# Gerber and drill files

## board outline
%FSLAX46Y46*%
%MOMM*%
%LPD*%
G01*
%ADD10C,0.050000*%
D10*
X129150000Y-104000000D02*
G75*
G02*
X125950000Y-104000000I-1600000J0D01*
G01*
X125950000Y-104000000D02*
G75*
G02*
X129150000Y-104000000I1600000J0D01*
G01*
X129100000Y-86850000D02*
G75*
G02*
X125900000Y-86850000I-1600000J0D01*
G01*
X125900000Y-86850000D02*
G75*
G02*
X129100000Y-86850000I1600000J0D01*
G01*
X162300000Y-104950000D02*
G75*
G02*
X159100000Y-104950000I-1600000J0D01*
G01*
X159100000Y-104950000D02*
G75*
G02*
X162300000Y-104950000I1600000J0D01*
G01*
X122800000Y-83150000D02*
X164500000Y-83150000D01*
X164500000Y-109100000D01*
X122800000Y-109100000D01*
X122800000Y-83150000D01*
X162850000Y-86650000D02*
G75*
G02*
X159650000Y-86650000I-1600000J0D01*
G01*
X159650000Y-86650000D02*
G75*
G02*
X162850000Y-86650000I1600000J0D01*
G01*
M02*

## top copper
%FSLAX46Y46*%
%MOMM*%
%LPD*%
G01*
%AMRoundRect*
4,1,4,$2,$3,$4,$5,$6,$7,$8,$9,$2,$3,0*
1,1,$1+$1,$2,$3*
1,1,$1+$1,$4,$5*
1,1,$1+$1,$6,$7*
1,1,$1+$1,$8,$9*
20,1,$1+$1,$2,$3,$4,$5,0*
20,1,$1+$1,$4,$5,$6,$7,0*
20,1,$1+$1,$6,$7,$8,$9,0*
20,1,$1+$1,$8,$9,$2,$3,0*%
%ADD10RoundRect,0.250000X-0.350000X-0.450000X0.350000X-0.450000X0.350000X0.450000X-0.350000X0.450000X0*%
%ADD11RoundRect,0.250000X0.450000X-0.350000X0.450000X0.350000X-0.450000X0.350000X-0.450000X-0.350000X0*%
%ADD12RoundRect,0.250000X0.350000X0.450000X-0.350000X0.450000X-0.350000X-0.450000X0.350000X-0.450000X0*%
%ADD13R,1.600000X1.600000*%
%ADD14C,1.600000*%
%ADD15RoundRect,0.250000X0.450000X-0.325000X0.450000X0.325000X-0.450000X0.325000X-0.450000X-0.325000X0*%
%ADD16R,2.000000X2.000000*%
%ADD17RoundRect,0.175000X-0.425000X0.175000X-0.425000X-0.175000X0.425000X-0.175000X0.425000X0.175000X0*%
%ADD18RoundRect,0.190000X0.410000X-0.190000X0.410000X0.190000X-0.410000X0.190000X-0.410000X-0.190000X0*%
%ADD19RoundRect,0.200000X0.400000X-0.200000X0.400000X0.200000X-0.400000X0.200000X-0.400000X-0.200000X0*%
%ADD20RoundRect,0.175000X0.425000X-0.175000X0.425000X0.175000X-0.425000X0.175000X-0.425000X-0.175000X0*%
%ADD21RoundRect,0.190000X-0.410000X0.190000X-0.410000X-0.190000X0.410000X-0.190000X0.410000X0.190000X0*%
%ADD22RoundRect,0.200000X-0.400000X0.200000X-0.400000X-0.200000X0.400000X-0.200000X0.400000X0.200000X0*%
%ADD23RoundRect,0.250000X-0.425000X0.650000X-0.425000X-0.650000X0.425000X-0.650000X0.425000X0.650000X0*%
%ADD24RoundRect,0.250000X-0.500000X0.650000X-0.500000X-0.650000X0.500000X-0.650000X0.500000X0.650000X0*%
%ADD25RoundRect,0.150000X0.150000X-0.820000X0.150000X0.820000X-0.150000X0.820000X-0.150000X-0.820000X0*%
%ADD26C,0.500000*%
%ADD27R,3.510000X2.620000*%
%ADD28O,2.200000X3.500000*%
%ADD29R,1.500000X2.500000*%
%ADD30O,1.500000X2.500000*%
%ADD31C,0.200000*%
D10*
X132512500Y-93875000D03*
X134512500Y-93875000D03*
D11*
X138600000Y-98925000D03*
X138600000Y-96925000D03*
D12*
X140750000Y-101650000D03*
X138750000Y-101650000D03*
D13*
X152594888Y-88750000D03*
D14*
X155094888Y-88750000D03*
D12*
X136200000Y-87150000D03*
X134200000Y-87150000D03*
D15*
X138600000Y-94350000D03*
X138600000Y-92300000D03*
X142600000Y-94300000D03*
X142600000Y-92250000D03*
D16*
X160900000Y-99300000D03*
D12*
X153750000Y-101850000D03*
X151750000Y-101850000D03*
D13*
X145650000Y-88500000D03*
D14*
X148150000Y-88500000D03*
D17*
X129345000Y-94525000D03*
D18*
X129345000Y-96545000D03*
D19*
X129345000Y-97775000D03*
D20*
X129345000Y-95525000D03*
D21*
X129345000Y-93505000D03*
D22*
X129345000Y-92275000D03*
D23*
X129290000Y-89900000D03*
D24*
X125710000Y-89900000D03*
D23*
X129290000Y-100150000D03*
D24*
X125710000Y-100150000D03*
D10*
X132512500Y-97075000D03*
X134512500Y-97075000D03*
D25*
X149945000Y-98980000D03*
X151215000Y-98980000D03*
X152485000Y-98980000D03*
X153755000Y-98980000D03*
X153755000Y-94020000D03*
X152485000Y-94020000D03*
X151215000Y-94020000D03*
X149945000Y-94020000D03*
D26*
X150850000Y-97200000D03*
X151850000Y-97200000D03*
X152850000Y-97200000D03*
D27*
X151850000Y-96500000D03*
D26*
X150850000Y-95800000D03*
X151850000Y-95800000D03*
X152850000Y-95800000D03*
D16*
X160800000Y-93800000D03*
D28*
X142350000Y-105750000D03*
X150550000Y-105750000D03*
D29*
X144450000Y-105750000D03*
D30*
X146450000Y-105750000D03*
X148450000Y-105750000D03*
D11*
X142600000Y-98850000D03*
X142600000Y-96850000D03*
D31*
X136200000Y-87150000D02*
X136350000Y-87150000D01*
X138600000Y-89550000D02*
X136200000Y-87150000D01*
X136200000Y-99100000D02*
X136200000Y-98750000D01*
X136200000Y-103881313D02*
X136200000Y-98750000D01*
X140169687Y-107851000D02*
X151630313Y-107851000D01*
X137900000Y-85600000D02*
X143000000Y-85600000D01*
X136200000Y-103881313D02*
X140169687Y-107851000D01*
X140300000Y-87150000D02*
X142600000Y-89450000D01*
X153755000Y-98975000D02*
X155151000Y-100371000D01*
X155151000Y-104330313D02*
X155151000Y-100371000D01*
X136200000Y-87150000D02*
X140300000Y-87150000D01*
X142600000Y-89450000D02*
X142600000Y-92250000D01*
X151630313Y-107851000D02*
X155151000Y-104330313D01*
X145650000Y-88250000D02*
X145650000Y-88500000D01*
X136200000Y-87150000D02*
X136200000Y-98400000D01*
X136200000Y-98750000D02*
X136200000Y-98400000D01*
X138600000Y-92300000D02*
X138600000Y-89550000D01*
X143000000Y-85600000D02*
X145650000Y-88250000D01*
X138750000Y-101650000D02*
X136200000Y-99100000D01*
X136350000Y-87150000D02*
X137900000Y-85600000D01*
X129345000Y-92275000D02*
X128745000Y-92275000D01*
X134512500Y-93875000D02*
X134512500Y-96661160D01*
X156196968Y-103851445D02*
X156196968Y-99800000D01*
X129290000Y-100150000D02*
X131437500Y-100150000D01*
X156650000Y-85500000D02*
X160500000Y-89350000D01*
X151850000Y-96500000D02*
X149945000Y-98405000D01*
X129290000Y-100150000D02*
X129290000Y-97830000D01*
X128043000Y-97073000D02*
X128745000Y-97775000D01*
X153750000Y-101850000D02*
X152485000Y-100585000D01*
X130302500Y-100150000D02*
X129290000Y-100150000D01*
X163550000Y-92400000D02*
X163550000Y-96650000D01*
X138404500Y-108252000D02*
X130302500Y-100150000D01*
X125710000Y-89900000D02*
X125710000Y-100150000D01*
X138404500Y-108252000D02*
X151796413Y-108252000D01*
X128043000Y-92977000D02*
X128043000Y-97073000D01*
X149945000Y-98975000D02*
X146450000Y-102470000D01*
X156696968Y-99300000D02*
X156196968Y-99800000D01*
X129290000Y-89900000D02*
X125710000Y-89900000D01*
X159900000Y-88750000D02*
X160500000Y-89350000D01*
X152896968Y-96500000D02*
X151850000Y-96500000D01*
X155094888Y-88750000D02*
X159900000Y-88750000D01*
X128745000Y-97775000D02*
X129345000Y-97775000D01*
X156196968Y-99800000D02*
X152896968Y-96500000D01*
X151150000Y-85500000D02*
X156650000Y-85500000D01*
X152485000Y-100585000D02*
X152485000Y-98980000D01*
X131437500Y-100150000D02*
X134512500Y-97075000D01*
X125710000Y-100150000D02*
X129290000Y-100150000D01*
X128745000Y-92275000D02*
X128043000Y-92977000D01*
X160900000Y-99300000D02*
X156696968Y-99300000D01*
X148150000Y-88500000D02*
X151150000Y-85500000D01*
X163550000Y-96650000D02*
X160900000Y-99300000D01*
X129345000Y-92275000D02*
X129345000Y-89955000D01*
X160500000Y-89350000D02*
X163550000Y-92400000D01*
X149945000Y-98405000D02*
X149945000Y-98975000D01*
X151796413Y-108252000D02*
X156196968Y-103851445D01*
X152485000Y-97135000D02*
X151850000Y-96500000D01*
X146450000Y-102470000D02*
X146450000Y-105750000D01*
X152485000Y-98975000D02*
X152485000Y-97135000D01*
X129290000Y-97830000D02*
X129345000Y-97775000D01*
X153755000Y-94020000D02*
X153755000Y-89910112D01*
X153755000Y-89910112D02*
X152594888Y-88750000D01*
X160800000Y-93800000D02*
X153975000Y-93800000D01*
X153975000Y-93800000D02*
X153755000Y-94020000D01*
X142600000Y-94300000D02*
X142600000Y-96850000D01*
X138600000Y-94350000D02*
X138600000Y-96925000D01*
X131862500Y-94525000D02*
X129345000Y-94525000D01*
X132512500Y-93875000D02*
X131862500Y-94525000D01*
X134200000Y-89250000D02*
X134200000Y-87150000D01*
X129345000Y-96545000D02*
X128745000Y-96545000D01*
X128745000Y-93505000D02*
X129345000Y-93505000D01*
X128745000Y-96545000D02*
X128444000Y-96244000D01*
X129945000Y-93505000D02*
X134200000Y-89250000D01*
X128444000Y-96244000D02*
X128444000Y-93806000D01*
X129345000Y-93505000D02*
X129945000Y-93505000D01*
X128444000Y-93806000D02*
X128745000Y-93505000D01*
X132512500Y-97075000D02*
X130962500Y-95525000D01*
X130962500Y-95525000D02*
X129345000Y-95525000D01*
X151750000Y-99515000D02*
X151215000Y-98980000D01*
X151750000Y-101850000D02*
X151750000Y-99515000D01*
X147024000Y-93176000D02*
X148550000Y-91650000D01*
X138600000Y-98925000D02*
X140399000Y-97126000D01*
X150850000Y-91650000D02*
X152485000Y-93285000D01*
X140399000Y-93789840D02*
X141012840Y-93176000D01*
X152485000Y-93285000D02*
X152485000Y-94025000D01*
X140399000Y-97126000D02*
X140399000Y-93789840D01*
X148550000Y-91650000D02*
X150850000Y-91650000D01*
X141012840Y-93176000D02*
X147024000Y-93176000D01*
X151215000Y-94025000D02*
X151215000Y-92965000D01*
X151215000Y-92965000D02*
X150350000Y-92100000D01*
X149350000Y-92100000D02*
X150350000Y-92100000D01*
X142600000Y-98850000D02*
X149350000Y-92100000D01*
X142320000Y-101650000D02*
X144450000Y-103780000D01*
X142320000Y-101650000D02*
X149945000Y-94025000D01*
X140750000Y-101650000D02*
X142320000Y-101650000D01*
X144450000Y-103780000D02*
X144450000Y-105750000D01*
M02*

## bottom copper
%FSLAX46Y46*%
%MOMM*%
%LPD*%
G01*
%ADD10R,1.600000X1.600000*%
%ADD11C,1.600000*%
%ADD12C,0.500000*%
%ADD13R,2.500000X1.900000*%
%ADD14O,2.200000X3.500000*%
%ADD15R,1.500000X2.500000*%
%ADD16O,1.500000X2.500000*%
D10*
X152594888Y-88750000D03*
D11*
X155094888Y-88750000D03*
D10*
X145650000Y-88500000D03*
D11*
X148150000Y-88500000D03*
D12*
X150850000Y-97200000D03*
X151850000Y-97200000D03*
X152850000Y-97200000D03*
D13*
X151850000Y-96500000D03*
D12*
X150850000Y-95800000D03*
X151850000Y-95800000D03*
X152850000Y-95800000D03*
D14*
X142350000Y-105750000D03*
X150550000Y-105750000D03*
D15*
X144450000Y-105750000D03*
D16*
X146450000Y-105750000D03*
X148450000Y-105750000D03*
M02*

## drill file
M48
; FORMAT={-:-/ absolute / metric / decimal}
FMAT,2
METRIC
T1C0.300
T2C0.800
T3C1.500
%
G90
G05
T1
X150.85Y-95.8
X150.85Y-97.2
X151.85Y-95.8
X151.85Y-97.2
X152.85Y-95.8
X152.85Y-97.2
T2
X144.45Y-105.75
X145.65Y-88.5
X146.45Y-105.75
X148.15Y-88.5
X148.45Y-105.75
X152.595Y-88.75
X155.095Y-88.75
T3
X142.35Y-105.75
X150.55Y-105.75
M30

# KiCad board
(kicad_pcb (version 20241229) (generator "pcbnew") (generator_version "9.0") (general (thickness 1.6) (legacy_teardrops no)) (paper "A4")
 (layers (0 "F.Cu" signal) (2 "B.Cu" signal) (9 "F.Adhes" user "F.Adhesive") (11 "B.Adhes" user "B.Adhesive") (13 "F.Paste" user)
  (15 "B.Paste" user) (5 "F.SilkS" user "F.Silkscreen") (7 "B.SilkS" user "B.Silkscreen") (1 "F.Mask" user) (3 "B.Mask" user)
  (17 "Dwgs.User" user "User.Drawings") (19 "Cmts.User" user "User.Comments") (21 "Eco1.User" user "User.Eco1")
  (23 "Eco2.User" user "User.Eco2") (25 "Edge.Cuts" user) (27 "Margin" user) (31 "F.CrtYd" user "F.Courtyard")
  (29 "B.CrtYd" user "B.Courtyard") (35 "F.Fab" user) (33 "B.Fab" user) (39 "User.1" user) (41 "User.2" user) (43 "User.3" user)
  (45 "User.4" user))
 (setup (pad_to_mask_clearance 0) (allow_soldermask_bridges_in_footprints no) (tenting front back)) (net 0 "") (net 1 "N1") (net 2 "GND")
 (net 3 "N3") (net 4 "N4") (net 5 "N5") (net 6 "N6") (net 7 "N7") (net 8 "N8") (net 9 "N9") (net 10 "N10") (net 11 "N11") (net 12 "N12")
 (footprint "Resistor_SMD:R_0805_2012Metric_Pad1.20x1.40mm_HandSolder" (layer "F.Cu") (at 133.5125 93.875)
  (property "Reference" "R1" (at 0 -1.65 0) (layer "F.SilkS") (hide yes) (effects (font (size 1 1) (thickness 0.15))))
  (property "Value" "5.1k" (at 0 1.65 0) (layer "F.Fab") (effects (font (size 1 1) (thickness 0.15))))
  (pad "1" smd roundrect (at -1 0) (size 1.2 1.4) (layers "F.Cu" "F.Mask" "F.Paste") (roundrect_rratio 0.208333) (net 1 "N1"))
  (pad "2" smd roundrect (at 1 0) (size 1.2 1.4) (layers "F.Cu" "F.Mask" "F.Paste") (roundrect_rratio 0.208333) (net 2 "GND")))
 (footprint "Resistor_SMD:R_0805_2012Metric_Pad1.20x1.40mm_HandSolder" (layer "F.Cu") (at 138.6 97.925 90)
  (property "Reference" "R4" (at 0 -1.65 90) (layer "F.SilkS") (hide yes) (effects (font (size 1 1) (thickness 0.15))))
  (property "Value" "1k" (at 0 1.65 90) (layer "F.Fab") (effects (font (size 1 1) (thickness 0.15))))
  (pad "1" smd roundrect (at -1 0 90) (size 1.2 1.4) (layers "F.Cu" "F.Mask" "F.Paste") (roundrect_rratio 0.208333) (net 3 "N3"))
  (pad "2" smd roundrect (at 1 0 90) (size 1.2 1.4) (layers "F.Cu" "F.Mask" "F.Paste") (roundrect_rratio 0.208333) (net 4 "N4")))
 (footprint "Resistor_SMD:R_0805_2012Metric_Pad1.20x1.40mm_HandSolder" (layer "F.Cu") (at 139.75 101.65 180)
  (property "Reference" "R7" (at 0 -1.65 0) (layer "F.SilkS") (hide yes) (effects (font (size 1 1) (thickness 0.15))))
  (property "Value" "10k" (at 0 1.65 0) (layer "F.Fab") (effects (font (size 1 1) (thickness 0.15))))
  (pad "1" smd roundrect (at -1 0 180) (size 1.2 1.4) (layers "F.Cu" "F.Mask" "F.Paste") (roundrect_rratio 0.208333) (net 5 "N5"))
  (pad "2" smd roundrect (at 1 0 180) (size 1.2 1.4) (layers "F.Cu" "F.Mask" "F.Paste") (roundrect_rratio 0.208333) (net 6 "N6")))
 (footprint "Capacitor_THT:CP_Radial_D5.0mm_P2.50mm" (layer "F.Cu") (at 152.594888 88.75)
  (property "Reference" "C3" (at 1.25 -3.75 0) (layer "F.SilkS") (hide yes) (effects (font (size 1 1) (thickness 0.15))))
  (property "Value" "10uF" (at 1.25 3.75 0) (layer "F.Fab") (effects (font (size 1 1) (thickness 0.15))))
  (pad "1" thru_hole rect (at 0 0) (size 1.6 1.6) (drill 0.8) (layers "*.Cu" "*.Mask") (remove_unused_layers no) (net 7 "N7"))
  (pad "2" thru_hole circle (at 2.5 0) (size 1.6 1.6) (drill 0.8) (layers "*.Cu" "*.Mask") (remove_unused_layers no) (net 2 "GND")))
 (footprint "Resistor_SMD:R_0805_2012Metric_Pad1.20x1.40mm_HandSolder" (layer "F.Cu") (at 135.2 87.15 180)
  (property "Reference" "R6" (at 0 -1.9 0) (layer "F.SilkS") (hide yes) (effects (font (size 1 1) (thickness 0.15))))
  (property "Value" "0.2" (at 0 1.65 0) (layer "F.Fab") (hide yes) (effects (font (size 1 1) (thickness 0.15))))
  (pad "1" smd roundrect (at -1 0 180) (size 1.2 1.4) (layers "F.Cu" "F.Mask" "F.Paste") (roundrect_rratio 0.208333) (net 6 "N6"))
  (pad "2" smd roundrect (at 1 0 180) (size 1.2 1.4) (layers "F.Cu" "F.Mask" "F.Paste") (roundrect_rratio 0.208333) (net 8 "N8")))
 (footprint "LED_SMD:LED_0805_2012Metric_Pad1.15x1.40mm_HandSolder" (layer "F.Cu") (at 138.6 93.325 90)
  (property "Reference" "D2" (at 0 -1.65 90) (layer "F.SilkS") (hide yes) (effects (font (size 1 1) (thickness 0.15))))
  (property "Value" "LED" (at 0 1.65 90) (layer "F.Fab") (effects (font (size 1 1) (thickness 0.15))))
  (pad "1" smd roundrect (at -1.025 0 90) (size 1.15 1.4) (layers "F.Cu" "F.Mask" "F.Paste") (roundrect_rratio 0.217391) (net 4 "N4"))
  (pad "2" smd roundrect (at 1.025 0 90) (size 1.15 1.4) (layers "F.Cu" "F.Mask" "F.Paste") (roundrect_rratio 0.217391) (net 6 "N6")))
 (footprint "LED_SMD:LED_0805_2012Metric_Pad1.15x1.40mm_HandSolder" (layer "F.Cu") (at 142.6 93.275 90)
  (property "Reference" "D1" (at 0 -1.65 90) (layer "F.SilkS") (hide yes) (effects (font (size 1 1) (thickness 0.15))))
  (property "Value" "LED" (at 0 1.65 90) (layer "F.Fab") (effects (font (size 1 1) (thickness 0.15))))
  (pad "1" smd roundrect (at -1.025 0 90) (size 1.15 1.4) (layers "F.Cu" "F.Mask" "F.Paste") (roundrect_rratio 0.217391) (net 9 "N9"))
  (pad "2" smd roundrect (at 1.025 0 90) (size 1.15 1.4) (layers "F.Cu" "F.Mask" "F.Paste") (roundrect_rratio 0.217391) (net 6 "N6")))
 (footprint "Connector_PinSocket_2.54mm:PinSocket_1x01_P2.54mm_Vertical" (layer "F.Cu") (at 160.9 99.3)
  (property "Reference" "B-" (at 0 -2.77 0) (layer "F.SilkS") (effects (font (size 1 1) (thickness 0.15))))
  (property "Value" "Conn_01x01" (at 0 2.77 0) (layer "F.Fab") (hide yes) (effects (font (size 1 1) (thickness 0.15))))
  (pad "1" smd rect (at 0 0) (size 2 2) (layers "F.Cu" "F.Mask" "F.Paste") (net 2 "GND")))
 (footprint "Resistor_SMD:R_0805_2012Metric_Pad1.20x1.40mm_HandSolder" (layer "F.Cu") (at 152.75 101.85 180)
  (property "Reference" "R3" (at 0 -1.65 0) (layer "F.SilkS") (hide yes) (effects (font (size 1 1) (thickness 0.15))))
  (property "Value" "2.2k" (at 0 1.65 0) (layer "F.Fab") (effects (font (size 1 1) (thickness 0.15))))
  (pad "1" smd roundrect (at -1 0 180) (size 1.2 1.4) (layers "F.Cu" "F.Mask" "F.Paste") (roundrect_rratio 0.208333) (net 2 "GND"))
  (pad "2" smd roundrect (at 1 0 180) (size 1.2 1.4) (layers "F.Cu" "F.Mask" "F.Paste") (roundrect_rratio 0.208333) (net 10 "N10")))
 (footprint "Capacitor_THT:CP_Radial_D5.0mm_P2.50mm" (layer "F.Cu") (at 145.65 88.5)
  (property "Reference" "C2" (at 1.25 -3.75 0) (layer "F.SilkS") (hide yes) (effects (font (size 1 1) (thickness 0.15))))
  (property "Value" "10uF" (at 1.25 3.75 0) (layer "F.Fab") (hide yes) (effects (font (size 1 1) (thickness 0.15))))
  (pad "1" thru_hole rect (at 0 0) (size 1.6 1.6) (drill 0.8) (layers "*.Cu" "*.Mask") (remove_unused_layers no) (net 6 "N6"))
  (pad "2" thru_hole circle (at 2.5 0) (size 1.6 1.6) (drill 0.8) (layers "*.Cu" "*.Mask") (remove_unused_layers no) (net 2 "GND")))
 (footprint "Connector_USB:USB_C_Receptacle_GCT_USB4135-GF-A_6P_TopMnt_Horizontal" (layer "F.Cu") (at 126.3125 95.025 -90)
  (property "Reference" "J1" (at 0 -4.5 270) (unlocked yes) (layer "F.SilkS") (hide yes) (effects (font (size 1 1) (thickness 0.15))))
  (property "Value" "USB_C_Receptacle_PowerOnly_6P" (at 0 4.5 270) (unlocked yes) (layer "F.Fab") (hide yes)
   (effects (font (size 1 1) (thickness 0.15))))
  (pad "A5" smd roundrect (at -0.5 -3.0325 270) (size 0.7 1.2) (layers "F.Cu" "F.Mask" "F.Paste") (roundrect_rratio 0.25) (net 1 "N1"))
  (pad "A9" smd roundrect (at 1.52 -3.0325 90) (size 0.76 1.2) (layers "F.Cu" "F.Mask" "F.Paste") (roundrect_rratio 0.25) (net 8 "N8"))
  (pad "A12" smd roundrect (at 2.75 -3.0325 90) (size 0.8 1.2) (layers "F.Cu" "F.Mask" "F.Paste") (roundrect_rratio 0.25) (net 2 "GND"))
  (pad "B5" smd roundrect (at 0.5 -3.0325 90) (size 0.7 1.2) (layers "F.Cu" "F.Mask" "F.Paste") (roundrect_rratio 0.25) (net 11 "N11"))
  (pad "B9" smd roundrect (at -1.52 -3.0325 270) (size 0.76 1.2) (layers "F.Cu" "F.Mask" "F.Paste") (roundrect_rratio 0.25) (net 8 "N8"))
  (pad "B12" smd roundrect (at -2.75 -3.0325 270) (size 0.8 1.2) (layers "F.Cu" "F.Mask" "F.Paste") (roundrect_rratio 0.25) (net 2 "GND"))
  (pad "S1" smd roundrect (at -5.125 -2.9775 270) (size 1.8 1.35) (layers "F.Cu" "F.Mask" "F.Paste") (roundrect_rratio 0.1851851852)
   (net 2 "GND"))
  (pad "S1" smd roundrect (at -5.125 0.6025 270) (size 1.8 1.5) (layers "F.Cu" "F.Mask" "F.Paste") (roundrect_rratio 0.1666666667)
   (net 2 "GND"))
  (pad "S1" smd roundrect (at 5.125 -2.9775 270) (size 1.8 1.35) (layers "F.Cu" "F.Mask" "F.Paste") (roundrect_rratio 0.1851851852)
   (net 2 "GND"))
  (pad "S1" smd roundrect (at 5.125 0.6025 270) (size 1.8 1.5) (layers "F.Cu" "F.Mask" "F.Paste") (roundrect_rratio 0.1666666667)
   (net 2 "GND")))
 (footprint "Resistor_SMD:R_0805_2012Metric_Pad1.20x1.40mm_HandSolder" (layer "F.Cu") (at 133.5125 97.075)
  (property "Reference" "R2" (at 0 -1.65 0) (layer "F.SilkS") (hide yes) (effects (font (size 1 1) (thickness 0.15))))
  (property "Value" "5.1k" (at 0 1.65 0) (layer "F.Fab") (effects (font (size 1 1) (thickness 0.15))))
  (pad "1" smd roundrect (at -1 0) (size 1.2 1.4) (layers "F.Cu" "F.Mask" "F.Paste") (roundrect_rratio 0.208333) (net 11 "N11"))
  (pad "2" smd roundrect (at 1 0) (size 1.2 1.4) (layers "F.Cu" "F.Mask" "F.Paste") (roundrect_rratio 0.208333) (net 2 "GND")))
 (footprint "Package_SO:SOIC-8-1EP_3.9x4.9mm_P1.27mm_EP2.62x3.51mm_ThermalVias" (layer "F.Cu") (at 151.85 96.5 90)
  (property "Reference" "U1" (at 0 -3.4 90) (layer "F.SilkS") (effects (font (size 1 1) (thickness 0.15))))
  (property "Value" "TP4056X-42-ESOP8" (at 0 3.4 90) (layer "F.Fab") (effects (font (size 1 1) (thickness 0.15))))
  (pad "" smd roundrect (at -0.655 -0.875 90) (size 1.1 1.47) (layers "F.Paste") (roundrect_rratio 0.227273))
  (pad "" smd roundrect (at -0.655 0.875 90) (size 1.1 1.47) (layers "F.Paste") (roundrect_rratio 0.227273))
  (pad "" smd roundrect (at 0.655 -0.875 90) (size 1.1 1.47) (layers "F.Paste") (roundrect_rratio 0.227273))
  (pad "" smd roundrect (at 0.655 0.875 90) (size 1.1 1.47) (layers "F.Paste") (roundrect_rratio 0.227273))
  (pad "1" smd roundrect (at -2.48 -1.905 90) (size 1.94 0.6) (layers "F.Cu" "F.Mask" "F.Paste") (roundrect_rratio 0.25) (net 2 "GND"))
  (pad "2" smd roundrect (at -2.48 -0.635 90) (size 1.94 0.6) (layers "F.Cu" "F.Mask" "F.Paste") (roundrect_rratio 0.25) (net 10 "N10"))
  (pad "3" smd roundrect (at -2.48 0.635 90) (size 1.94 0.6) (layers "F.Cu" "F.Mask" "F.Paste") (roundrect_rratio 0.25) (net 2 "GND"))
  (pad "4" smd roundrect (at -2.48 1.905 90) (size 1.94 0.6) (layers "F.Cu" "F.Mask" "F.Paste") (roundrect_rratio 0.25) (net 6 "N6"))
  (pad "5" smd roundrect (at 2.48 1.905 90) (size 1.94 0.6) (layers "F.Cu" "F.Mask" "F.Paste") (roundrect_rratio 0.25) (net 7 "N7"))
  (pad "6" smd roundrect (at 2.48 0.635 90) (size 1.94 0.6) (layers "F.Cu" "F.Mask" "F.Paste") (roundrect_rratio 0.25) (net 3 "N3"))
  (pad "7" smd roundrect (at 2.48 -0.635 90) (size 1.94 0.6) (layers "F.Cu" "F.Mask" "F.Paste") (roundrect_rratio 0.25) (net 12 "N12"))
  (pad "8" smd roundrect (at 2.48 -1.905 90) (size 1.94 0.6) (layers "F.Cu" "F.Mask" "F.Paste") (roundrect_rratio 0.25) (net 5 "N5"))
  (pad "9" thru_hole circle (at -0.7 -1 90) (size 0.5 0.5) (drill 0.3) (layers "*.Cu") (remove_unused_layers no) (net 2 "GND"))
  (pad "9" thru_hole circle (at -0.7 0 90) (size 0.5 0.5) (drill 0.3) (layers "*.Cu") (remove_unused_layers no) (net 2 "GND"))
  (pad "9" thru_hole circle (at -0.7 1 90) (size 0.5 0.5) (drill 0.3) (layers "*.Cu") (remove_unused_layers no) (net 2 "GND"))
  (pad "9" smd rect (at 0 0 90) (size 1.9 2.5) (layers "B.Cu") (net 2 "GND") (zone_connect 2))
  (pad "9" smd rect (at 0 0 90) (size 2.62 3.51) (layers "F.Cu" "F.Mask") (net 2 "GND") (zone_connect 2))
  (pad "9" thru_hole circle (at 0.7 -1 90) (size 0.5 0.5) (drill 0.3) (layers "*.Cu") (remove_unused_layers no) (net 2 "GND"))
  (pad "9" thru_hole circle (at 0.7 0 90) (size 0.5 0.5) (drill 0.3) (layers "*.Cu") (remove_unused_layers no) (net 2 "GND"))
  (pad "9" thru_hole circle (at 0.7 1 90) (size 0.5 0.5) (drill 0.3) (layers "*.Cu") (remove_unused_layers no) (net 2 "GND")))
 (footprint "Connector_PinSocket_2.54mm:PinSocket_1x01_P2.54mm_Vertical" (layer "F.Cu") (at 160.8 93.8)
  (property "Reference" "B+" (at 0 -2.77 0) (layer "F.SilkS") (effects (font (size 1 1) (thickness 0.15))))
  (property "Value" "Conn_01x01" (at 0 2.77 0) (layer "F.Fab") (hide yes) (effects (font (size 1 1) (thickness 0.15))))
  (pad "1" smd rect (at 0 0) (size 2 2) (layers "F.Cu" "F.Mask" "F.Paste") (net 7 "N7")))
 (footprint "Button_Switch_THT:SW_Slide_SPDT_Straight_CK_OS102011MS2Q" (layer "F.Cu") (at 144.45 105.75)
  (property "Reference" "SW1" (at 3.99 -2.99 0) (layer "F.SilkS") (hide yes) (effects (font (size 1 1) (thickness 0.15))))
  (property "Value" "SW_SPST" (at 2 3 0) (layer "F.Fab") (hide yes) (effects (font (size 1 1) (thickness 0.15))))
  (pad "" thru_hole oval (at -2.1 0) (size 2.2 3.5) (drill 1.5) (layers "*.Cu" "*.Mask") (remove_unused_layers no))
  (pad "" thru_hole oval (at 6.1 0) (size 2.2 3.5) (drill 1.5) (layers "*.Cu" "*.Mask") (remove_unused_layers no))
  (pad "1" thru_hole rect (at 0 0) (size 1.5 2.5) (drill 0.8) (layers "*.Cu" "*.Mask") (remove_unused_layers no) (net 5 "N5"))
  (pad "2" thru_hole oval (at 2 0) (size 1.5 2.5) (drill 0.8) (layers "*.Cu" "*.Mask") (remove_unused_layers no) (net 2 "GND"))
  (pad "3" thru_hole oval (at 4 0) (size 1.5 2.5) (drill 0.8) (layers "*.Cu" "*.Mask") (remove_unused_layers no)))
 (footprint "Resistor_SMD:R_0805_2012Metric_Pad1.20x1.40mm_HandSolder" (layer "F.Cu") (at 142.6 97.85 90)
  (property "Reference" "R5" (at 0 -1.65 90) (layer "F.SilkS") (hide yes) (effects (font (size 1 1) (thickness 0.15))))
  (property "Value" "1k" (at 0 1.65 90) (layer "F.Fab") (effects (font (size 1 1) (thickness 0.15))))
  (pad "1" smd roundrect (at -1 0 90) (size 1.2 1.4) (layers "F.Cu" "F.Mask" "F.Paste") (roundrect_rratio 0.208333) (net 12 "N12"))
  (pad "2" smd roundrect (at 1 0 90) (size 1.2 1.4) (layers "F.Cu" "F.Mask" "F.Paste") (roundrect_rratio 0.208333) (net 9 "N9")))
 (gr_circle (center 127.55 104) (end 127.55 105.6) (stroke (width 0.05) (type default)) (fill no) (layer "Edge.Cuts"))
 (gr_circle (center 127.5 86.85) (end 127.5 88.45) (stroke (width 0.05) (type default)) (fill no) (layer "Edge.Cuts"))
 (gr_circle (center 160.7 104.95) (end 160.7 106.55) (stroke (width 0.05) (type default)) (fill no) (layer "Edge.Cuts"))
 (gr_rect (start 122.8 83.15) (end 164.5 109.1) (stroke (width 0.05) (type default)) (fill no) (layer "Edge.Cuts"))
 (gr_circle (center 161.25 86.65) (end 161.25 88.25) (stroke (width 0.05) (type default)) (fill no) (layer "Edge.Cuts"))
 (segment (start 136.2 87.15) (end 136.35 87.15) (width 0.2) (layer "F.Cu") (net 6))
 (segment (start 138.6 89.55) (end 136.2 87.15) (width 0.2) (layer "F.Cu") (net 6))
 (segment (start 136.2 99.1) (end 136.2 98.75) (width 0.2) (layer "F.Cu") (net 6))
 (segment (start 136.2 103.881313) (end 136.2 98.75) (width 0.2) (layer "F.Cu") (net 6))
 (segment (start 140.169687 107.851) (end 151.630313 107.851) (width 0.2) (layer "F.Cu") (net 6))
 (segment (start 137.9 85.6) (end 143 85.6) (width 0.2) (layer "F.Cu") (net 6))
 (segment (start 136.2 103.881313) (end 140.169687 107.851) (width 0.2) (layer "F.Cu") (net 6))
 (segment (start 140.3 87.15) (end 142.6 89.45) (width 0.2) (layer "F.Cu") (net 6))
 (segment (start 153.755 98.975) (end 155.151 100.371) (width 0.2) (layer "F.Cu") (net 6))
 (segment (start 155.151 104.330313) (end 155.151 100.371) (width 0.2) (layer "F.Cu") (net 6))
 (segment (start 136.2 87.15) (end 140.3 87.15) (width 0.2) (layer "F.Cu") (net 6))
 (segment (start 142.6 89.45) (end 142.6 92.25) (width 0.2) (layer "F.Cu") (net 6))
 (segment (start 151.630313 107.851) (end 155.151 104.330313) (width 0.2) (layer "F.Cu") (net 6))
 (segment (start 145.65 88.25) (end 145.65 88.5) (width 0.2) (layer "F.Cu") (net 6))
 (segment (start 136.2 87.15) (end 136.2 98.4) (width 0.2) (layer "F.Cu") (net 6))
 (segment (start 136.2 98.75) (end 136.2 98.4) (width 0.2) (layer "F.Cu") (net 6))
 (segment (start 138.6 92.3) (end 138.6 89.55) (width 0.2) (layer "F.Cu") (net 6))
 (segment (start 143 85.6) (end 145.65 88.25) (width 0.2) (layer "F.Cu") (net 6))
 (segment (start 138.75 101.65) (end 136.2 99.1) (width 0.2) (layer "F.Cu") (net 6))
 (segment (start 136.35 87.15) (end 137.9 85.6) (width 0.2) (layer "F.Cu") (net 6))
 (segment (start 129.345 92.275) (end 128.745 92.275) (width 0.2) (layer "F.Cu") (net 2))
 (segment (start 134.5125 93.875) (end 134.5125 96.66116) (width 0.2) (layer "F.Cu") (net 2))
 (segment (start 156.196968 103.851445) (end 156.196968 99.8) (width 0.2) (layer "F.Cu") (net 2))
 (segment (start 129.29 100.15) (end 131.4375 100.15) (width 0.2) (layer "F.Cu") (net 2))
 (segment (start 156.65 85.5) (end 160.5 89.35) (width 0.2) (layer "F.Cu") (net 2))
 (segment (start 151.85 96.5) (end 149.945 98.405) (width 0.2) (layer "F.Cu") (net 2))
 (segment (start 129.29 100.15) (end 129.29 97.83) (width 0.2) (layer "F.Cu") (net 2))
 (segment (start 128.043 97.073) (end 128.745 97.775) (width 0.2) (layer "F.Cu") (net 2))
 (segment (start 153.75 101.85) (end 152.485 100.585) (width 0.2) (layer "F.Cu") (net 2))
 (segment (start 130.3025 100.15) (end 129.29 100.15) (width 0.2) (layer "F.Cu") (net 2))
 (segment (start 163.55 92.4) (end 163.55 96.65) (width 0.2) (layer "F.Cu") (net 2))
 (segment (start 138.4045 108.252) (end 130.3025 100.15) (width 0.2) (layer "F.Cu") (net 2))
 (segment (start 125.71 89.9) (end 125.71 100.15) (width 0.2) (layer "F.Cu") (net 2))
 (segment (start 138.4045 108.252) (end 151.796413 108.252) (width 0.2) (layer "F.Cu") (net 2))
 (segment (start 128.043 92.977) (end 128.043 97.073) (width 0.2) (layer "F.Cu") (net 2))
 (segment (start 149.945 98.975) (end 146.45 102.47) (width 0.2) (layer "F.Cu") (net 2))
 (segment (start 156.696968 99.3) (end 156.196968 99.8) (width 0.2) (layer "F.Cu") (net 2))
 (segment (start 129.29 89.9) (end 125.71 89.9) (width 0.2) (layer "F.Cu") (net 2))
 (segment (start 159.9 88.75) (end 160.5 89.35) (width 0.2) (layer "F.Cu") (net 2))
 (segment (start 152.896968 96.5) (end 151.85 96.5) (width 0.2) (layer "F.Cu") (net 2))
 (segment (start 155.094888 88.75) (end 159.9 88.75) (width 0.2) (layer "F.Cu") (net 2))
 (segment (start 128.745 97.775) (end 129.345 97.775) (width 0.2) (layer "F.Cu") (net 2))
 (segment (start 156.196968 99.8) (end 152.896968 96.5) (width 0.2) (layer "F.Cu") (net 2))
 (segment (start 151.15 85.5) (end 156.65 85.5) (width 0.2) (layer "F.Cu") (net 2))
 (segment (start 152.485 100.585) (end 152.485 98.98) (width 0.2) (layer "F.Cu") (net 2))
 (segment (start 131.4375 100.15) (end 134.5125 97.075) (width 0.2) (layer "F.Cu") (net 2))
 (segment (start 125.71 100.15) (end 129.29 100.15) (width 0.2) (layer "F.Cu") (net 2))
 (segment (start 128.745 92.275) (end 128.043 92.977) (width 0.2) (layer "F.Cu") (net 2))
 (segment (start 160.9 99.3) (end 156.696968 99.3) (width 0.2) (layer "F.Cu") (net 2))
 (segment (start 148.15 88.5) (end 151.15 85.5) (width 0.2) (layer "F.Cu") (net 2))
 (segment (start 163.55 96.65) (end 160.9 99.3) (width 0.2) (layer "F.Cu") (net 2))
 (segment (start 129.345 92.275) (end 129.345 89.955) (width 0.2) (layer "F.Cu") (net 2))
 (segment (start 160.5 89.35) (end 163.55 92.4) (width 0.2) (layer "F.Cu") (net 2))
 (segment (start 149.945 98.405) (end 149.945 98.975) (width 0.2) (layer "F.Cu") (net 2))
 (segment (start 151.796413 108.252) (end 156.196968 103.851445) (width 0.2) (layer "F.Cu") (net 2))
 (segment (start 152.485 97.135) (end 151.85 96.5) (width 0.2) (layer "F.Cu") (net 2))
 (segment (start 146.45 102.47) (end 146.45 105.75) (width 0.2) (layer "F.Cu") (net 2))
 (segment (start 152.485 98.975) (end 152.485 97.135) (width 0.2) (layer "F.Cu") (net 2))
 (segment (start 129.29 97.83) (end 129.345 97.775) (width 0.2) (layer "F.Cu") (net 2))
 (segment (start 153.755 94.02) (end 153.755 89.910112) (width 0.2) (layer "F.Cu") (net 7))
 (segment (start 153.755 89.910112) (end 152.594888 88.75) (width 0.2) (layer "F.Cu") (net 7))
 (segment (start 160.8 93.8) (end 153.975 93.8) (width 0.2) (layer "F.Cu") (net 7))
 (segment (start 153.975 93.8) (end 153.755 94.02) (width 0.2) (layer "F.Cu") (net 7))
 (segment (start 142.6 94.3) (end 142.6 96.85) (width 0.2) (layer "F.Cu") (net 9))
 (segment (start 138.6 94.35) (end 138.6 96.925) (width 0.2) (layer "F.Cu") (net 4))
 (segment (start 131.8625 94.525) (end 129.345 94.525) (width 0.2) (layer "F.Cu") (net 1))
 (segment (start 132.5125 93.875) (end 131.8625 94.525) (width 0.2) (layer "F.Cu") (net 1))
 (segment (start 134.2 89.25) (end 134.2 87.15) (width 0.2) (layer "F.Cu") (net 8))
 (segment (start 129.345 96.545) (end 128.745 96.545) (width 0.2) (layer "F.Cu") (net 8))
 (segment (start 128.745 93.505) (end 129.345 93.505) (width 0.2) (layer "F.Cu") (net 8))
 (segment (start 128.745 96.545) (end 128.444 96.244) (width 0.2) (layer "F.Cu") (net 8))
 (segment (start 129.945 93.505) (end 134.2 89.25) (width 0.2) (layer "F.Cu") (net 8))
 (segment (start 128.444 96.244) (end 128.444 93.806) (width 0.2) (layer "F.Cu") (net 8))
 (segment (start 129.345 93.505) (end 129.945 93.505) (width 0.2) (layer "F.Cu") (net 8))
 (segment (start 128.444 93.806) (end 128.745 93.505) (width 0.2) (layer "F.Cu") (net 8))
 (segment (start 132.5125 97.075) (end 130.9625 95.525) (width 0.2) (layer "F.Cu") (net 11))
 (segment (start 130.9625 95.525) (end 129.345 95.525) (width 0.2) (layer "F.Cu") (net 11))
 (segment (start 151.75 99.515) (end 151.215 98.98) (width 0.2) (layer "F.Cu") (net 10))
 (segment (start 151.75 101.85) (end 151.75 99.515) (width 0.2) (layer "F.Cu") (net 10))
 (segment (start 147.024 93.176) (end 148.55 91.65) (width 0.2) (layer "F.Cu") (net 3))
 (segment (start 138.6 98.925) (end 140.399 97.126) (width 0.2) (layer "F.Cu") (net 3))
 (segment (start 150.85 91.65) (end 152.485 93.285) (width 0.2) (layer "F.Cu") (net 3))
 (segment (start 140.399 93.78984) (end 141.01284 93.176) (width 0.2) (layer "F.Cu") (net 3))
 (segment (start 152.485 93.285) (end 152.485 94.025) (width 0.2) (layer "F.Cu") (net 3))
 (segment (start 140.399 97.126) (end 140.399 93.78984) (width 0.2) (layer "F.Cu") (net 3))
 (segment (start 148.55 91.65) (end 150.85 91.65) (width 0.2) (layer "F.Cu") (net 3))
 (segment (start 141.01284 93.176) (end 147.024 93.176) (width 0.2) (layer "F.Cu") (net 3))
 (segment (start 151.215 94.025) (end 151.215 92.965) (width 0.2) (layer "F.Cu") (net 12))
 (segment (start 151.215 92.965) (end 150.35 92.1) (width 0.2) (layer "F.Cu") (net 12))
 (segment (start 149.35 92.1) (end 150.35 92.1) (width 0.2) (layer "F.Cu") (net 12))
 (segment (start 142.6 98.85) (end 149.35 92.1) (width 0.2) (layer "F.Cu") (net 12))
 (segment (start 142.32 101.65) (end 144.45 103.78) (width 0.2) (layer "F.Cu") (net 5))
 (segment (start 142.32 101.65) (end 149.945 94.025) (width 0.2) (layer "F.Cu") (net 5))
 (segment (start 140.75 101.65) (end 142.32 101.65) (width 0.2) (layer "F.Cu") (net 5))
 (segment (start 144.45 103.78) (end 144.45 105.75) (width 0.2) (layer "F.Cu") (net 5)))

